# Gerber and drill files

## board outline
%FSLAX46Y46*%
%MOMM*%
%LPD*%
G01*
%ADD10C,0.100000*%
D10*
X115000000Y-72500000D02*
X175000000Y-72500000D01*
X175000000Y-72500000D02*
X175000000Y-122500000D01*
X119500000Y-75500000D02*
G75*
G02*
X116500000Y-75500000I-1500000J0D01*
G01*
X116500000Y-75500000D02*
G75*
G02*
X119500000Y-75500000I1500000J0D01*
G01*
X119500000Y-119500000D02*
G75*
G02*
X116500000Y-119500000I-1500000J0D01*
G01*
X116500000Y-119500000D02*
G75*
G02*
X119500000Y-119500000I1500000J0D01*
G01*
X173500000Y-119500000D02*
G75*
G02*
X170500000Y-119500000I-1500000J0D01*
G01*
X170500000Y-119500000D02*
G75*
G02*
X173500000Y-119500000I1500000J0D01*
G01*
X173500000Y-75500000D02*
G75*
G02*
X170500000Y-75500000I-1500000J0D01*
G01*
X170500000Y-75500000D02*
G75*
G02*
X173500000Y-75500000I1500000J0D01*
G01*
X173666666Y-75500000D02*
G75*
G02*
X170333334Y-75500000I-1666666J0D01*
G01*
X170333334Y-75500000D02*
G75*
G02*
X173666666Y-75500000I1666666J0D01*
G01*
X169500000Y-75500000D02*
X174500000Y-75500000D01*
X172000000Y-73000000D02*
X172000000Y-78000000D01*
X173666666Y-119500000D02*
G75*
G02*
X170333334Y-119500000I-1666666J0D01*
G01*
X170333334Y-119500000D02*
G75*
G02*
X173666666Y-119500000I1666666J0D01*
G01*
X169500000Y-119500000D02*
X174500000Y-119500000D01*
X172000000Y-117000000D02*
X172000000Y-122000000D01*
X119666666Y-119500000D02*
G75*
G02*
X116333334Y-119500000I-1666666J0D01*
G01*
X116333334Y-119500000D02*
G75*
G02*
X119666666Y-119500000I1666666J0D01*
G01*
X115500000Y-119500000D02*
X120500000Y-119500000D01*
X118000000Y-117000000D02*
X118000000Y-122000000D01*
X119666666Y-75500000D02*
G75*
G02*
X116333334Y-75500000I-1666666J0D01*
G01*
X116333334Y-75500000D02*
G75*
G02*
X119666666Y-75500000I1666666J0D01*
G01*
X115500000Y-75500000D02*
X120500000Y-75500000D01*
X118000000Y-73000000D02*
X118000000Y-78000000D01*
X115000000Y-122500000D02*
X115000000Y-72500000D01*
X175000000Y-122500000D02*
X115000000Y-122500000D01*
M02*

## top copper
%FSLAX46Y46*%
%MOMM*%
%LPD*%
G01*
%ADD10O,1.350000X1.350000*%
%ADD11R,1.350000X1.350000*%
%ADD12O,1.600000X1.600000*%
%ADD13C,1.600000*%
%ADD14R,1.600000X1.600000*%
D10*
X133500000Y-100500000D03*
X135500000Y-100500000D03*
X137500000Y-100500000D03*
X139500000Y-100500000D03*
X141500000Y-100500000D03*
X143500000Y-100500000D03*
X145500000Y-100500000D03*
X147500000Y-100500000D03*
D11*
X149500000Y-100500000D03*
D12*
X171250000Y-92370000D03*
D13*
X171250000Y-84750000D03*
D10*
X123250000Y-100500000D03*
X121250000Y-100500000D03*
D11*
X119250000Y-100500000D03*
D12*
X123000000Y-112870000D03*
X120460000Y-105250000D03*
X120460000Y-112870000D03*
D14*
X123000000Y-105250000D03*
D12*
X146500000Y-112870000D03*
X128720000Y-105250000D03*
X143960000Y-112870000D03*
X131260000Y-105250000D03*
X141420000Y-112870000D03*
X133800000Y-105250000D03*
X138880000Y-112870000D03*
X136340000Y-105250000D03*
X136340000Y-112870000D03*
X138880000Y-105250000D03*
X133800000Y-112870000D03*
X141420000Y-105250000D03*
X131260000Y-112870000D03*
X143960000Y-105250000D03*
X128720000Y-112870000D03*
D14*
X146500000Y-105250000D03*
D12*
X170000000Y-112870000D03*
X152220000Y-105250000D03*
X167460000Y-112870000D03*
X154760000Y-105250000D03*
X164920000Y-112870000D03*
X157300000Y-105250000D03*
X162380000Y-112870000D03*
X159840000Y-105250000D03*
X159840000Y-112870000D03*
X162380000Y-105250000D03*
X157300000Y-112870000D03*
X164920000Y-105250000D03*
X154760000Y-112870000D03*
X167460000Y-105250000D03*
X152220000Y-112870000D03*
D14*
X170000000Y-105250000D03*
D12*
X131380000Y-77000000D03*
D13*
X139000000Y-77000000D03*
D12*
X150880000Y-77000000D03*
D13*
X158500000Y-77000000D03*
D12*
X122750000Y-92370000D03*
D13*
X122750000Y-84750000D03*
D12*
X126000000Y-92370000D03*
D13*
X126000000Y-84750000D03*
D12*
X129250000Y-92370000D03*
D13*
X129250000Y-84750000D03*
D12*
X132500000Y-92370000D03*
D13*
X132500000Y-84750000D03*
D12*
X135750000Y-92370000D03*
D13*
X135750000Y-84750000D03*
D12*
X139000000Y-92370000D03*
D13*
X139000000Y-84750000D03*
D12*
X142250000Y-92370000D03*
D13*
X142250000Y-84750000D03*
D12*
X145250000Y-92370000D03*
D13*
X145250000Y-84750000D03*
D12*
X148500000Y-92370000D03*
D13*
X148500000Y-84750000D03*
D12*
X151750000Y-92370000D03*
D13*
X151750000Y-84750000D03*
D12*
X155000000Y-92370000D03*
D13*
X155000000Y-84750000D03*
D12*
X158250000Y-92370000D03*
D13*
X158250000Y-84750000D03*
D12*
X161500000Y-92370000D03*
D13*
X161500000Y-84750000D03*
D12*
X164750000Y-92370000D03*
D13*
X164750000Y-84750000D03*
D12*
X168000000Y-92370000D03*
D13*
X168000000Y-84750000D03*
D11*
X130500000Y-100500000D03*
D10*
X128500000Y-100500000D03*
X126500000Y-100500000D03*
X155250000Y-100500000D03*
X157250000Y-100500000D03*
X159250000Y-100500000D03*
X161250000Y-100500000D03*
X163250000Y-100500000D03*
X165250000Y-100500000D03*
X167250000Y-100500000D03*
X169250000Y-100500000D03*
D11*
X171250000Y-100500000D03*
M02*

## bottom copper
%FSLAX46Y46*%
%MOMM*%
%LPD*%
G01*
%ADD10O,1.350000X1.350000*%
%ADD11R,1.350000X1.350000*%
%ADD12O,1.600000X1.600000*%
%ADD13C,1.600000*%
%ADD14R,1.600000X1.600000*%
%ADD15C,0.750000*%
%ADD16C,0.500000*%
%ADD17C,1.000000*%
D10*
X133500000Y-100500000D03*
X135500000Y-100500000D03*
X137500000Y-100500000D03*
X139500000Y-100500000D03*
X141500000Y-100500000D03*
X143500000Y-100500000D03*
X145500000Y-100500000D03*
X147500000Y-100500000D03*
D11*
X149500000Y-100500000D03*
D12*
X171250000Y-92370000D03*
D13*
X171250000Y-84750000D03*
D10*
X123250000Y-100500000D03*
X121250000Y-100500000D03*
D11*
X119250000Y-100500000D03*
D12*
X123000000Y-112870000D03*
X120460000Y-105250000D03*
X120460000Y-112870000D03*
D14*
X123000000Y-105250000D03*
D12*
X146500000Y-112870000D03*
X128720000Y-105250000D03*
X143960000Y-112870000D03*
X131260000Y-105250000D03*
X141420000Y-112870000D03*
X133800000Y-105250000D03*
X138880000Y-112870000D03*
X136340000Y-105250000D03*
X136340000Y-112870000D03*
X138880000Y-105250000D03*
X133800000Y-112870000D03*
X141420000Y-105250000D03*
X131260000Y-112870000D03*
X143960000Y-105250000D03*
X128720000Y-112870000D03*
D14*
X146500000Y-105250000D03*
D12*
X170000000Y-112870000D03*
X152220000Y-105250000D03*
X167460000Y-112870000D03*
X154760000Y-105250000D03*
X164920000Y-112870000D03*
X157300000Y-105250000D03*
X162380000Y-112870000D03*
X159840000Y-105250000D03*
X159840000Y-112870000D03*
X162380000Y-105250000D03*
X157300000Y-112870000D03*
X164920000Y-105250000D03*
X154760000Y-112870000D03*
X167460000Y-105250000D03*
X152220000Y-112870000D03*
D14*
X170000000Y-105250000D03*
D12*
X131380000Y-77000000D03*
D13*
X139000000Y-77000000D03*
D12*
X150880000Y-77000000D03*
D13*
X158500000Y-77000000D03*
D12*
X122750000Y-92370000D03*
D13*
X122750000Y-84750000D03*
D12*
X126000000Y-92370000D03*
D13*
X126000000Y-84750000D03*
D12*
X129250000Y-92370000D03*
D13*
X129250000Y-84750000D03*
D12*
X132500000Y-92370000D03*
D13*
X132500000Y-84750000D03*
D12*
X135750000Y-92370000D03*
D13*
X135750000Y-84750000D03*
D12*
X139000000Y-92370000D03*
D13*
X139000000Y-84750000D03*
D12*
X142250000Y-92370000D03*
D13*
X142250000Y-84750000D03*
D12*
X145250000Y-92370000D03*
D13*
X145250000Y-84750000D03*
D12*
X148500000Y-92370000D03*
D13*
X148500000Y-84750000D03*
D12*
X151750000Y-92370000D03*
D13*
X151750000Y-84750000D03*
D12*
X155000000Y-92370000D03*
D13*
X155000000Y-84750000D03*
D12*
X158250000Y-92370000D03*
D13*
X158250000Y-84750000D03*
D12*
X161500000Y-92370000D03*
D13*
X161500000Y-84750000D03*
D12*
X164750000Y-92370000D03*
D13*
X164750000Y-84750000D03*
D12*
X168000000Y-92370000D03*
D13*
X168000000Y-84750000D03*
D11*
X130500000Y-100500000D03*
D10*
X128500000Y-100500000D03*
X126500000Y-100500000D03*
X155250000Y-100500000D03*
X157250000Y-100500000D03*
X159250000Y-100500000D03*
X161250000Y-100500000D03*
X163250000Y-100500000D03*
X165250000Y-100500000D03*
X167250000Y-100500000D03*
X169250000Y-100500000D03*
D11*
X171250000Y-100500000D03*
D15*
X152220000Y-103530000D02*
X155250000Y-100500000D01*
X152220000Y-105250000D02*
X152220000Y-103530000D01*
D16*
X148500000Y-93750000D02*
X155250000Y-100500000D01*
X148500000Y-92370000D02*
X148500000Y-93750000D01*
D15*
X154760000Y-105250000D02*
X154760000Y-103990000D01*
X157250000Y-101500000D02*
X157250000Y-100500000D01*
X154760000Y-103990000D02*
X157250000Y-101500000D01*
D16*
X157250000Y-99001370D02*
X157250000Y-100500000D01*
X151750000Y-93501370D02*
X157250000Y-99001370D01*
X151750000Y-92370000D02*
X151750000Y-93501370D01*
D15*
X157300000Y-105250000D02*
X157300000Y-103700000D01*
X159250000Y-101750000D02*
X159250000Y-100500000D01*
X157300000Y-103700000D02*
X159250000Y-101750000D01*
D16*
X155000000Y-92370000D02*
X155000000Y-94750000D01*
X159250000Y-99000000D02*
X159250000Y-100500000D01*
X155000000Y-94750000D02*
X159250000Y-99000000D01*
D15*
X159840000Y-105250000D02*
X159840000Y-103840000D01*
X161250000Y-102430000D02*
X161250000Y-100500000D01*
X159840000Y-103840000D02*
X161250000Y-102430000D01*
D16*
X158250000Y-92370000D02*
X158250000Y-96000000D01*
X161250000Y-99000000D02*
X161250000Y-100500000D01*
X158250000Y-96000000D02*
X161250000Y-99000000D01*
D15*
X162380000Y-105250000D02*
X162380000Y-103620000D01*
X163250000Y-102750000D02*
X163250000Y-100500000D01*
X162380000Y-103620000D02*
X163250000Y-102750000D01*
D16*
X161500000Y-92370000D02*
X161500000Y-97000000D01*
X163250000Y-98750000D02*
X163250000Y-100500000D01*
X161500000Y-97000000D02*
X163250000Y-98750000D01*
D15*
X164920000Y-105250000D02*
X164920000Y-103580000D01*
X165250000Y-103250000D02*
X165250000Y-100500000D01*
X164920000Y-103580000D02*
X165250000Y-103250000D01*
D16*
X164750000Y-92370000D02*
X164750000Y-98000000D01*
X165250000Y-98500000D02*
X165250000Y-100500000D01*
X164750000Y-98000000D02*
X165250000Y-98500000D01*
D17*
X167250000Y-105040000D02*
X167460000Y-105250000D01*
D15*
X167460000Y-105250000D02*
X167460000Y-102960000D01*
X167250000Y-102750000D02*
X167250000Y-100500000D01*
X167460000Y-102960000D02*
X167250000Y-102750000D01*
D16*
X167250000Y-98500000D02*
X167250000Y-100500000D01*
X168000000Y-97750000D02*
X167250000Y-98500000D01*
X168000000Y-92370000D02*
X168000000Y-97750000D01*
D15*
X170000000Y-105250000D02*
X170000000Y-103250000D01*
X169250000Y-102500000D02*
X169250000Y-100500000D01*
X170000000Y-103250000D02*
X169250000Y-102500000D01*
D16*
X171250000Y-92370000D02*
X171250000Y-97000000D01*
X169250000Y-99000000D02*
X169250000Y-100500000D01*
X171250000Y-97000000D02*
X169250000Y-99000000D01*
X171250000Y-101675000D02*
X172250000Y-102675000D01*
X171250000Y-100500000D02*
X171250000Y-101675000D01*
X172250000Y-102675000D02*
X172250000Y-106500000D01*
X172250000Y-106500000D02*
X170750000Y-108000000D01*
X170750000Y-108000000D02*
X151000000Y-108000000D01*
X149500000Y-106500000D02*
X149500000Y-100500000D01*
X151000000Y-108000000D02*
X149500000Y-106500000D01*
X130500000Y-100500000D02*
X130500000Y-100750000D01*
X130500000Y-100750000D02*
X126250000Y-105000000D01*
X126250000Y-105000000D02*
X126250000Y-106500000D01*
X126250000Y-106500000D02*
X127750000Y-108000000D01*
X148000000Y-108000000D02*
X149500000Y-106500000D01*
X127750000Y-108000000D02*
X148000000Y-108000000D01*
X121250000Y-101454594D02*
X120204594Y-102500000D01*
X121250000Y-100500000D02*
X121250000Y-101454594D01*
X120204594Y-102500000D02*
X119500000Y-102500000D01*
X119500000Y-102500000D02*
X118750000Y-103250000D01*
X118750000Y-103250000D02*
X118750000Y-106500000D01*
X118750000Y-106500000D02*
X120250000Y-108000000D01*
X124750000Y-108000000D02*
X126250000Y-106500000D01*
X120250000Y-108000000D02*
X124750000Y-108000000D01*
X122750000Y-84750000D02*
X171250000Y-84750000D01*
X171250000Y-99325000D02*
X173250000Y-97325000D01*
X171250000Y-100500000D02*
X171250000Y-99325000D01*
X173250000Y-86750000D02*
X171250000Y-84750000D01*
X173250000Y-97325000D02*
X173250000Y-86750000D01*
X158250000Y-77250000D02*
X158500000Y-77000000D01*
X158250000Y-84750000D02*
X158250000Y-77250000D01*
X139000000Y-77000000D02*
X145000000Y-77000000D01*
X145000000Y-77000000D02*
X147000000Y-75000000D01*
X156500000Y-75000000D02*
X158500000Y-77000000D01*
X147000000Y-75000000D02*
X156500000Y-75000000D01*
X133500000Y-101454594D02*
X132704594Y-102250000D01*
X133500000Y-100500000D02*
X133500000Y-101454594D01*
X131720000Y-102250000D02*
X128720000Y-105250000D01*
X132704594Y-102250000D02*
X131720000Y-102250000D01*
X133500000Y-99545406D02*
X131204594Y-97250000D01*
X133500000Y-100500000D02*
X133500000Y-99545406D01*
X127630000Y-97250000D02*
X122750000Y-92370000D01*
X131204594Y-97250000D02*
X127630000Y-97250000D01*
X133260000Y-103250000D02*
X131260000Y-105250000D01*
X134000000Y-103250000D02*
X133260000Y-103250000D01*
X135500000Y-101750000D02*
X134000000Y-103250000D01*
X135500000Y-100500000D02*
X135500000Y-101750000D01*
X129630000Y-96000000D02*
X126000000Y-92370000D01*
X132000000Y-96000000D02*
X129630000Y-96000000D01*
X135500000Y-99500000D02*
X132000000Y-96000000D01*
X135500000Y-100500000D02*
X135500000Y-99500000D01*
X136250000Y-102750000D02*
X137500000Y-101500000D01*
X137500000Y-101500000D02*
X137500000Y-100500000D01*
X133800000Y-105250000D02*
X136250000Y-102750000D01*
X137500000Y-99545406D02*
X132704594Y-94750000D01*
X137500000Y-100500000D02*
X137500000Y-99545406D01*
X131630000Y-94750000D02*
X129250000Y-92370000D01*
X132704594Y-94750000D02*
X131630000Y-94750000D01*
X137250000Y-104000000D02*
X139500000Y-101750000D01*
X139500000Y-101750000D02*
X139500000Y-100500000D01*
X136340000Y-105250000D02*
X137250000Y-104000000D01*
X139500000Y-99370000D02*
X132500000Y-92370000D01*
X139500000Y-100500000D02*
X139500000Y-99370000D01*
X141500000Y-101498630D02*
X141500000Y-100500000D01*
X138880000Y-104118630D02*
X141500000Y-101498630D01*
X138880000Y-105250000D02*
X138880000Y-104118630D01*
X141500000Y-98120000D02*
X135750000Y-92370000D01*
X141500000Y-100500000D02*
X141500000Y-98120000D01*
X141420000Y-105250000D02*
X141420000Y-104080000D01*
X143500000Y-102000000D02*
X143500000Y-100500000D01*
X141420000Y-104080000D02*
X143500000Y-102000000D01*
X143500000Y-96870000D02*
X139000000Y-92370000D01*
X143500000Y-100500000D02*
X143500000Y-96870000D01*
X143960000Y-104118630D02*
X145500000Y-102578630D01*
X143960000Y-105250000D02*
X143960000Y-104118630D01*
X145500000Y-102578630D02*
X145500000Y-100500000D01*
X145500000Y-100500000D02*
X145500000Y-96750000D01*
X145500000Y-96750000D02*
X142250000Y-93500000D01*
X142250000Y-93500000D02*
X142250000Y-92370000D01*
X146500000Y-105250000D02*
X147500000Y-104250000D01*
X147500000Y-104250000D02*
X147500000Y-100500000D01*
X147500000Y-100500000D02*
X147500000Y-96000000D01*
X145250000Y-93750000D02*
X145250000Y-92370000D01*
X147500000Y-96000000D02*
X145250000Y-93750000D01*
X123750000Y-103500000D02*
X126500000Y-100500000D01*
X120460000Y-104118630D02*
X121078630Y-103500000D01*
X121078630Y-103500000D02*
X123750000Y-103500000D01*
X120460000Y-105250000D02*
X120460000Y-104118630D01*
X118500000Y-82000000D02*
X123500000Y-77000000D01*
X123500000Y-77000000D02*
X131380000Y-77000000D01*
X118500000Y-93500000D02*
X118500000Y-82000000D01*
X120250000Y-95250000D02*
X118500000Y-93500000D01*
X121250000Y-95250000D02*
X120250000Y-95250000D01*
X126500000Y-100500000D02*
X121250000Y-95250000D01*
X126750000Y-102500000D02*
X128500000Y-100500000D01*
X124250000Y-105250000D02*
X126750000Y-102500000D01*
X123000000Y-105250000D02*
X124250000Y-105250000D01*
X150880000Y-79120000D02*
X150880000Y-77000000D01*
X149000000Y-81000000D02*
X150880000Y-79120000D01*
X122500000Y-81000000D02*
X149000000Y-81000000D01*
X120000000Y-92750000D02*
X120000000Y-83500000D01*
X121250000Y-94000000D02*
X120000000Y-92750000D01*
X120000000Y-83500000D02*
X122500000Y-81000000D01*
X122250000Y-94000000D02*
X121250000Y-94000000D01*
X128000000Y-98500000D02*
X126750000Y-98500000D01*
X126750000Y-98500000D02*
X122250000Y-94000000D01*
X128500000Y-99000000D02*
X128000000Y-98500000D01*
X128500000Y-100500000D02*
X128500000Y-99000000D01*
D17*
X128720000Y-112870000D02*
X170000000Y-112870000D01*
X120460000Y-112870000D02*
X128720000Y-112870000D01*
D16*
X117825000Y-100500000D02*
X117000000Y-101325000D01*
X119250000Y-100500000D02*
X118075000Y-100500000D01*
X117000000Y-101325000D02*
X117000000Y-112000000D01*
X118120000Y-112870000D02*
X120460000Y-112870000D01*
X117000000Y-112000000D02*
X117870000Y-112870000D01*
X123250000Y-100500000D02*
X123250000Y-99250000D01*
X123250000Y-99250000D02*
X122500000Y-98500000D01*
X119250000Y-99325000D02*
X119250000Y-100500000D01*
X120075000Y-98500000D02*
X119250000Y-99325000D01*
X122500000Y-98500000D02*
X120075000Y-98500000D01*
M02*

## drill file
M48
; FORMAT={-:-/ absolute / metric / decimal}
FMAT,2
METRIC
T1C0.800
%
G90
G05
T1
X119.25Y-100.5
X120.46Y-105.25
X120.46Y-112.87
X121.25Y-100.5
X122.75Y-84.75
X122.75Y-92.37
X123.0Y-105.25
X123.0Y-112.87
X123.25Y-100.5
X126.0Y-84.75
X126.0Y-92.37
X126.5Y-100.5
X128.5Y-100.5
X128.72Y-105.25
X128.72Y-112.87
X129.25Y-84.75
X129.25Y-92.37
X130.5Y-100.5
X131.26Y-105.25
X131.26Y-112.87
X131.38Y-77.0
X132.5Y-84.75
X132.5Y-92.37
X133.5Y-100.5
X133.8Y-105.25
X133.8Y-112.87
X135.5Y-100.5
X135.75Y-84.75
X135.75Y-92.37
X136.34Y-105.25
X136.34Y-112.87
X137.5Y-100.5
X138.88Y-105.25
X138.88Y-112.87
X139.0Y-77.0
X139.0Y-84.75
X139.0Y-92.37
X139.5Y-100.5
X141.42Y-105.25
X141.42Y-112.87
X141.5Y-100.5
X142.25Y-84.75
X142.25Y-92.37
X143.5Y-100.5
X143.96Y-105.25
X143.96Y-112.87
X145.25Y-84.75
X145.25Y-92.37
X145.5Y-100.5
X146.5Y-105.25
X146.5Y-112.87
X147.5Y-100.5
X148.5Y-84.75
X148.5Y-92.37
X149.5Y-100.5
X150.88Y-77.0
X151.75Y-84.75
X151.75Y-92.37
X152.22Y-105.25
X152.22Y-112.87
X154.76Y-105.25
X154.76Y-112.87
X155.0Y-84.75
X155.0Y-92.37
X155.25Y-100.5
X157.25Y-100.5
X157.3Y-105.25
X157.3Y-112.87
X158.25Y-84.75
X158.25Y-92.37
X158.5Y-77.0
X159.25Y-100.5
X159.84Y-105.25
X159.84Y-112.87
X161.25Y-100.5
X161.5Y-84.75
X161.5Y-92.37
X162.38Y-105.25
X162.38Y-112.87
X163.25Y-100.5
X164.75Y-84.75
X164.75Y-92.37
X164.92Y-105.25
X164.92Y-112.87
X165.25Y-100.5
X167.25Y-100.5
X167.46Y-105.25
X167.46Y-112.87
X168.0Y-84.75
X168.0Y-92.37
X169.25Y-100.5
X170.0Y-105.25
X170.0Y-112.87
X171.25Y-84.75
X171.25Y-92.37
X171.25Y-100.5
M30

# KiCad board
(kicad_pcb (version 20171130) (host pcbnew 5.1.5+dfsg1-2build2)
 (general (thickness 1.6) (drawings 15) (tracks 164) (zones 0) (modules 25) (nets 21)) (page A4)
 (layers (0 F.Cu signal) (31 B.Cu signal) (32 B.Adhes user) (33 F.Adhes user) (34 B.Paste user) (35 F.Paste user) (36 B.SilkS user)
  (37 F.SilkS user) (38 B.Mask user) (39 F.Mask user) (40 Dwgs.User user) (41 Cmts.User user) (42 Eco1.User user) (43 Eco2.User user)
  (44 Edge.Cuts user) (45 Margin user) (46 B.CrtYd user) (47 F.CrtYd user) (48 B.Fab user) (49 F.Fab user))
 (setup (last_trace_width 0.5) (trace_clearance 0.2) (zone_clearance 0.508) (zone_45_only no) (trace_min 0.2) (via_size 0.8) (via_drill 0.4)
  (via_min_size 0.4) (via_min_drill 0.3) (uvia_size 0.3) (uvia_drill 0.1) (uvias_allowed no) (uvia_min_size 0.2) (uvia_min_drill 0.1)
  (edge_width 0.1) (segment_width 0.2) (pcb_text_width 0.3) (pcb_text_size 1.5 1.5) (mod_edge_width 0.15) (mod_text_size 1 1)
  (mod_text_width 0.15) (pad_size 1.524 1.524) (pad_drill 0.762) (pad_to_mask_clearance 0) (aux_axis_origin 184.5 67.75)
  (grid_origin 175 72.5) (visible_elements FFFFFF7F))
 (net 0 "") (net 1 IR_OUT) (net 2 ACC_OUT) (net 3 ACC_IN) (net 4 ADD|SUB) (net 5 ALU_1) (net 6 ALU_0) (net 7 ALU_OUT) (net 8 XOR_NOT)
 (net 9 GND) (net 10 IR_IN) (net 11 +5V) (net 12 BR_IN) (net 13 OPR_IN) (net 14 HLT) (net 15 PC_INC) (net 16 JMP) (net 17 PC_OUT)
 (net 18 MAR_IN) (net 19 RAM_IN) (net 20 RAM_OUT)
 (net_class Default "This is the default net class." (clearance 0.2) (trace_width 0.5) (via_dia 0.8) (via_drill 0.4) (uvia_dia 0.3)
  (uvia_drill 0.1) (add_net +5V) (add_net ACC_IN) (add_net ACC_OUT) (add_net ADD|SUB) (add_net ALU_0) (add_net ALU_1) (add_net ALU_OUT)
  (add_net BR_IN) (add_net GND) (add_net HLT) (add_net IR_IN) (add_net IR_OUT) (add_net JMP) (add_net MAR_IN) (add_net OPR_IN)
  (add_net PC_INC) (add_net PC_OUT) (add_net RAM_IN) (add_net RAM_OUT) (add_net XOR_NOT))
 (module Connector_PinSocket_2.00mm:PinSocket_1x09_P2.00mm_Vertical (layer F.Cu) (at 149.5 100.5 270)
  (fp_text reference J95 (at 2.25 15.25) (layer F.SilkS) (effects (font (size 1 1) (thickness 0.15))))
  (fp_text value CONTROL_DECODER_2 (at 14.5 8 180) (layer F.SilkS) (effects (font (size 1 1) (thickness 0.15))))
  (pad 9 thru_hole oval (at 0 16 270) (size 1.35 1.35) (drill 0.8) (layers *.Cu *.Mask) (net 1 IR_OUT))
  (pad 8 thru_hole oval (at 0 14 270) (size 1.35 1.35) (drill 0.8) (layers *.Cu *.Mask) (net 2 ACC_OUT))
  (pad 7 thru_hole oval (at 0 12 270) (size 1.35 1.35) (drill 0.8) (layers *.Cu *.Mask) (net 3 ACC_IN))
  (pad 6 thru_hole oval (at 0 10 270) (size 1.35 1.35) (drill 0.8) (layers *.Cu *.Mask) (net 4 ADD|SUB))
  (pad 5 thru_hole oval (at 0 8 270) (size 1.35 1.35) (drill 0.8) (layers *.Cu *.Mask) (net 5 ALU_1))
  (pad 4 thru_hole oval (at 0 6 270) (size 1.35 1.35) (drill 0.8) (layers *.Cu *.Mask) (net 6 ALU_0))
  (pad 3 thru_hole oval (at 0 4 270) (size 1.35 1.35) (drill 0.8) (layers *.Cu *.Mask) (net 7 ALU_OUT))
  (pad 2 thru_hole oval (at 0 2 270) (size 1.35 1.35) (drill 0.8) (layers *.Cu *.Mask) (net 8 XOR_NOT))
  (pad 1 thru_hole rect (at 0 0 270) (size 1.35 1.35) (drill 0.8) (layers *.Cu *.Mask) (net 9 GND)))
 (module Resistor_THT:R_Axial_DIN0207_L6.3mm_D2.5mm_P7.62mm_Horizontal (layer F.Cu) (at 171.25 84.75 270)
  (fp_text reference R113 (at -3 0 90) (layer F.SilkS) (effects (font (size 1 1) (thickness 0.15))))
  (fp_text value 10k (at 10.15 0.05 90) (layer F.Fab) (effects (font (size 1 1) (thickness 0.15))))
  (pad 2 thru_hole oval (at 7.62 0 270) (size 1.6 1.6) (drill 0.8) (layers *.Cu *.Mask) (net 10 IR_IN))
  (pad 1 thru_hole circle (at 0 0 270) (size 1.6 1.6) (drill 0.8) (layers *.Cu *.Mask) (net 9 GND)))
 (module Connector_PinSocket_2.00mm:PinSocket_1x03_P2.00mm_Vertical (layer F.Cu) (at 119.25 100.5 90)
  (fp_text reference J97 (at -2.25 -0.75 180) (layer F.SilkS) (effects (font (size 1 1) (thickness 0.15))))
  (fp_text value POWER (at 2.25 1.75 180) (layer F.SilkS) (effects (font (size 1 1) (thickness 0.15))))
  (pad 3 thru_hole oval (at 0 4 90) (size 1.35 1.35) (drill 0.8) (layers *.Cu *.Mask) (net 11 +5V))
  (pad 2 thru_hole oval (at 0 2 90) (size 1.35 1.35) (drill 0.8) (layers *.Cu *.Mask) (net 9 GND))
  (pad 1 thru_hole rect (at 0 0 90) (size 1.35 1.35) (drill 0.8) (layers *.Cu *.Mask) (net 11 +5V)))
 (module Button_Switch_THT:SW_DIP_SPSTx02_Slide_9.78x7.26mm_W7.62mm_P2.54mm (layer F.Cu) (at 123 105.25 270)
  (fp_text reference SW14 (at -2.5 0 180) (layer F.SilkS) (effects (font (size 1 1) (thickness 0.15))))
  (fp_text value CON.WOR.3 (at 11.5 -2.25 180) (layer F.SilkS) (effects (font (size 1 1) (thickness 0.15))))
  (pad 4 thru_hole oval (at 7.62 0 270) (size 1.6 1.6) (drill 0.8) (layers *.Cu *.Mask) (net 11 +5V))
  (pad 2 thru_hole oval (at 0 2.54 270) (size 1.6 1.6) (drill 0.8) (layers *.Cu *.Mask) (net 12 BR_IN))
  (pad 3 thru_hole oval (at 7.62 2.54 270) (size 1.6 1.6) (drill 0.8) (layers *.Cu *.Mask) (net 11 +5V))
  (pad 1 thru_hole rect (at 0 0 270) (size 1.6 1.6) (drill 0.8) (layers *.Cu *.Mask) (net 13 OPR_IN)))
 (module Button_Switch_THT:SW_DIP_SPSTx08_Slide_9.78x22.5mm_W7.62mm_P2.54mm (layer F.Cu) (at 146.5 105.25 270)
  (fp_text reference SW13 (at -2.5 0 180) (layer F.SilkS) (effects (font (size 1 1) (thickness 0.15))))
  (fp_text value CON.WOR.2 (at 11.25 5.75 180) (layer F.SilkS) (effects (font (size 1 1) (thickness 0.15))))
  (pad 16 thru_hole oval (at 7.62 0 270) (size 1.6 1.6) (drill 0.8) (layers *.Cu *.Mask) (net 11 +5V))
  (pad 8 thru_hole oval (at 0 17.78 270) (size 1.6 1.6) (drill 0.8) (layers *.Cu *.Mask) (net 1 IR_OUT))
  (pad 15 thru_hole oval (at 7.62 2.54 270) (size 1.6 1.6) (drill 0.8) (layers *.Cu *.Mask) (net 11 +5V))
  (pad 7 thru_hole oval (at 0 15.24 270) (size 1.6 1.6) (drill 0.8) (layers *.Cu *.Mask) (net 2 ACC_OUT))
  (pad 14 thru_hole oval (at 7.62 5.08 270) (size 1.6 1.6) (drill 0.8) (layers *.Cu *.Mask) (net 11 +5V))
  (pad 6 thru_hole oval (at 0 12.7 270) (size 1.6 1.6) (drill 0.8) (layers *.Cu *.Mask) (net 3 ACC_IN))
  (pad 13 thru_hole oval (at 7.62 7.62 270) (size 1.6 1.6) (drill 0.8) (layers *.Cu *.Mask) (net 11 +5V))
  (pad 5 thru_hole oval (at 0 10.16 270) (size 1.6 1.6) (drill 0.8) (layers *.Cu *.Mask) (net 4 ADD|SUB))
  (pad 12 thru_hole oval (at 7.62 10.16 270) (size 1.6 1.6) (drill 0.8) (layers *.Cu *.Mask) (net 11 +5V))
  (pad 4 thru_hole oval (at 0 7.62 270) (size 1.6 1.6) (drill 0.8) (layers *.Cu *.Mask) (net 5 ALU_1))
  (pad 11 thru_hole oval (at 7.62 12.7 270) (size 1.6 1.6) (drill 0.8) (layers *.Cu *.Mask) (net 11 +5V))
  (pad 3 thru_hole oval (at 0 5.08 270) (size 1.6 1.6) (drill 0.8) (layers *.Cu *.Mask) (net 6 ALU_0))
  (pad 10 thru_hole oval (at 7.62 15.24 270) (size 1.6 1.6) (drill 0.8) (layers *.Cu *.Mask) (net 11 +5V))
  (pad 2 thru_hole oval (at 0 2.54 270) (size 1.6 1.6) (drill 0.8) (layers *.Cu *.Mask) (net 7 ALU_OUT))
  (pad 9 thru_hole oval (at 7.62 17.78 270) (size 1.6 1.6) (drill 0.8) (layers *.Cu *.Mask) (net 11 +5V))
  (pad 1 thru_hole rect (at 0 0 270) (size 1.6 1.6) (drill 0.8) (layers *.Cu *.Mask) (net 8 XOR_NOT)))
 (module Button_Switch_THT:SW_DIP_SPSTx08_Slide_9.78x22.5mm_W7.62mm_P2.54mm (layer F.Cu) (at 170 105.25 270)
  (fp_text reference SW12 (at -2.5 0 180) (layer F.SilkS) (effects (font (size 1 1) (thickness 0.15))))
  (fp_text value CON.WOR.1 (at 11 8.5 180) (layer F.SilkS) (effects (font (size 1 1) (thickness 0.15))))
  (pad 16 thru_hole oval (at 7.62 0 270) (size 1.6 1.6) (drill 0.8) (layers *.Cu *.Mask) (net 11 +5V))
  (pad 8 thru_hole oval (at 0 17.78 270) (size 1.6 1.6) (drill 0.8) (layers *.Cu *.Mask) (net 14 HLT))
  (pad 15 thru_hole oval (at 7.62 2.54 270) (size 1.6 1.6) (drill 0.8) (layers *.Cu *.Mask) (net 11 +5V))
  (pad 7 thru_hole oval (at 0 15.24 270) (size 1.6 1.6) (drill 0.8) (layers *.Cu *.Mask) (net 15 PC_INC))
  (pad 14 thru_hole oval (at 7.62 5.08 270) (size 1.6 1.6) (drill 0.8) (layers *.Cu *.Mask) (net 11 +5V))
  (pad 6 thru_hole oval (at 0 12.7 270) (size 1.6 1.6) (drill 0.8) (layers *.Cu *.Mask) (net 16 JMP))
  (pad 13 thru_hole oval (at 7.62 7.62 270) (size 1.6 1.6) (drill 0.8) (layers *.Cu *.Mask) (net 11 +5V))
  (pad 5 thru_hole oval (at 0 10.16 270) (size 1.6 1.6) (drill 0.8) (layers *.Cu *.Mask) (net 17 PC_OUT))
  (pad 12 thru_hole oval (at 7.62 10.16 270) (size 1.6 1.6) (drill 0.8) (layers *.Cu *.Mask) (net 11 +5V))
  (pad 4 thru_hole oval (at 0 7.62 270) (size 1.6 1.6) (drill 0.8) (layers *.Cu *.Mask) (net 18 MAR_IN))
  (pad 11 thru_hole oval (at 7.62 12.7 270) (size 1.6 1.6) (drill 0.8) (layers *.Cu *.Mask) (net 11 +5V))
  (pad 3 thru_hole oval (at 0 5.08 270) (size 1.6 1.6) (drill 0.8) (layers *.Cu *.Mask) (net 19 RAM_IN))
  (pad 10 thru_hole oval (at 7.62 15.24 270) (size 1.6 1.6) (drill 0.8) (layers *.Cu *.Mask) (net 11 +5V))
  (pad 2 thru_hole oval (at 0 2.54 270) (size 1.6 1.6) (drill 0.8) (layers *.Cu *.Mask) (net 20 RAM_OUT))
  (pad 9 thru_hole oval (at 7.62 17.78 270) (size 1.6 1.6) (drill 0.8) (layers *.Cu *.Mask) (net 11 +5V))
  (pad 1 thru_hole rect (at 0 0 270) (size 1.6 1.6) (drill 0.8) (layers *.Cu *.Mask) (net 10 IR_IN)))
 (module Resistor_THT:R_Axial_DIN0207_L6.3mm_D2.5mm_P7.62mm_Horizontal (layer F.Cu) (at 139 77 180)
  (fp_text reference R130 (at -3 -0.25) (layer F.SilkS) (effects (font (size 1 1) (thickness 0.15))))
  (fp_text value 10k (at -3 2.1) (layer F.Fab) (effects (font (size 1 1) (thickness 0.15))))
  (pad 2 thru_hole oval (at 7.62 0 180) (size 1.6 1.6) (drill 0.8) (layers *.Cu *.Mask) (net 12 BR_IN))
  (pad 1 thru_hole circle (at 0 0 180) (size 1.6 1.6) (drill 0.8) (layers *.Cu *.Mask) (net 9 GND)))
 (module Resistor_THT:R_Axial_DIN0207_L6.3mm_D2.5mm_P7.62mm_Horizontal (layer F.Cu) (at 158.5 77 180)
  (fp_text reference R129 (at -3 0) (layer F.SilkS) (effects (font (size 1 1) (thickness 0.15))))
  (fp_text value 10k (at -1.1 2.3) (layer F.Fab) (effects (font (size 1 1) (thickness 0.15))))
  (pad 2 thru_hole oval (at 7.62 0 180) (size 1.6 1.6) (drill 0.8) (layers *.Cu *.Mask) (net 13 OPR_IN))
  (pad 1 thru_hole circle (at 0 0 180) (size 1.6 1.6) (drill 0.8) (layers *.Cu *.Mask) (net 9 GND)))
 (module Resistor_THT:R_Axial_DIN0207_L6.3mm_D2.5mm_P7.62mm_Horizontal (layer F.Cu) (at 122.75 84.75 270)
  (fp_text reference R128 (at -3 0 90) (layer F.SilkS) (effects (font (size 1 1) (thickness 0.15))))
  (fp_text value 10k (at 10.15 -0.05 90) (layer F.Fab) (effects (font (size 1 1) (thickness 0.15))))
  (pad 2 thru_hole oval (at 7.62 0 270) (size 1.6 1.6) (drill 0.8) (layers *.Cu *.Mask) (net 1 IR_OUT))
  (pad 1 thru_hole circle (at 0 0 270) (size 1.6 1.6) (drill 0.8) (layers *.Cu *.Mask) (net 9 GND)))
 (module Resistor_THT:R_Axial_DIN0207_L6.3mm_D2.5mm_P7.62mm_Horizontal (layer F.Cu) (at 126 84.75 270)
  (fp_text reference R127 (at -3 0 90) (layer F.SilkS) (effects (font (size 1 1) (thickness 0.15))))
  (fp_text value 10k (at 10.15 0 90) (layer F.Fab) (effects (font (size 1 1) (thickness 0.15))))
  (pad 2 thru_hole oval (at 7.62 0 270) (size 1.6 1.6) (drill 0.8) (layers *.Cu *.Mask) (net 2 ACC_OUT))
  (pad 1 thru_hole circle (at 0 0 270) (size 1.6 1.6) (drill 0.8) (layers *.Cu *.Mask) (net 9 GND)))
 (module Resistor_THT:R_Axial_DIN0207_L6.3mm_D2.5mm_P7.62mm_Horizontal (layer F.Cu) (at 129.25 84.75 270)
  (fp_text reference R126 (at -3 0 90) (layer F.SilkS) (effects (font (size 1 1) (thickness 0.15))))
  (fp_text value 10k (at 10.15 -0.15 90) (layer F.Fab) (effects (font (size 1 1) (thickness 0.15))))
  (pad 2 thru_hole oval (at 7.62 0 270) (size 1.6 1.6) (drill 0.8) (layers *.Cu *.Mask) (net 3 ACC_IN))
  (pad 1 thru_hole circle (at 0 0 270) (size 1.6 1.6) (drill 0.8) (layers *.Cu *.Mask) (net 9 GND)))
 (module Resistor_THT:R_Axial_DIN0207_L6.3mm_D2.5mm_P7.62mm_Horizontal (layer F.Cu) (at 132.5 84.75 270)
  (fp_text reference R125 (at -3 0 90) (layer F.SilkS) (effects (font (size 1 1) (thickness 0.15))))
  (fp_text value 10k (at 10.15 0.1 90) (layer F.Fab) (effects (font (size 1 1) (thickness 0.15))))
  (pad 2 thru_hole oval (at 7.62 0 270) (size 1.6 1.6) (drill 0.8) (layers *.Cu *.Mask) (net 4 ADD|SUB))
  (pad 1 thru_hole circle (at 0 0 270) (size 1.6 1.6) (drill 0.8) (layers *.Cu *.Mask) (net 9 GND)))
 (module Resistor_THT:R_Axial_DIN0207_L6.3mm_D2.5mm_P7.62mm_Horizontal (layer F.Cu) (at 135.75 84.75 270)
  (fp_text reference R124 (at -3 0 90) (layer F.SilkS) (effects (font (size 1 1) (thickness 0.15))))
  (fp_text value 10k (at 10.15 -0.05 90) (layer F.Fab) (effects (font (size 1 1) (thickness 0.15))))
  (pad 2 thru_hole oval (at 7.62 0 270) (size 1.6 1.6) (drill 0.8) (layers *.Cu *.Mask) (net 5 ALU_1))
  (pad 1 thru_hole circle (at 0 0 270) (size 1.6 1.6) (drill 0.8) (layers *.Cu *.Mask) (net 9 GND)))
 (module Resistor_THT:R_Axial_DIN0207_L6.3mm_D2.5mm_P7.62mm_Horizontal (layer F.Cu) (at 139 84.75 270)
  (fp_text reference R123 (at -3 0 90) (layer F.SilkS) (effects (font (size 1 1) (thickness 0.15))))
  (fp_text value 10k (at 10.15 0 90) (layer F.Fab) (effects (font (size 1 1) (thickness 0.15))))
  (pad 2 thru_hole oval (at 7.62 0 270) (size 1.6 1.6) (drill 0.8) (layers *.Cu *.Mask) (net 6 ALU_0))
  (pad 1 thru_hole circle (at 0 0 270) (size 1.6 1.6) (drill 0.8) (layers *.Cu *.Mask) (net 9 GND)))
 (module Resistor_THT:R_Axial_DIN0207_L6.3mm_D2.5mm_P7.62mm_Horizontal (layer F.Cu) (at 142.25 84.75 270)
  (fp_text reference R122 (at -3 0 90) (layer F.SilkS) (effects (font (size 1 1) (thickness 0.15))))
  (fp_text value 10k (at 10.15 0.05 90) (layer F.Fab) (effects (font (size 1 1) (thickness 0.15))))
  (pad 2 thru_hole oval (at 7.62 0 270) (size 1.6 1.6) (drill 0.8) (layers *.Cu *.Mask) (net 7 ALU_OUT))
  (pad 1 thru_hole circle (at 0 0 270) (size 1.6 1.6) (drill 0.8) (layers *.Cu *.Mask) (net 9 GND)))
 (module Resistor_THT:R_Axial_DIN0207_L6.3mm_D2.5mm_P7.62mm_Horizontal (layer F.Cu) (at 145.25 84.75 270)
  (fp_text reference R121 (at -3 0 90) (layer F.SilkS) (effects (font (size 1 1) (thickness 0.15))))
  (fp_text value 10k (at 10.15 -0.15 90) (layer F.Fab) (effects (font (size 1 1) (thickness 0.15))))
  (pad 2 thru_hole oval (at 7.62 0 270) (size 1.6 1.6) (drill 0.8) (layers *.Cu *.Mask) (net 8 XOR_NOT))
  (pad 1 thru_hole circle (at 0 0 270) (size 1.6 1.6) (drill 0.8) (layers *.Cu *.Mask) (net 9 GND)))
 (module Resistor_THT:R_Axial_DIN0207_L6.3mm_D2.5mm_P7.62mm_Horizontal (layer F.Cu) (at 148.5 84.75 270)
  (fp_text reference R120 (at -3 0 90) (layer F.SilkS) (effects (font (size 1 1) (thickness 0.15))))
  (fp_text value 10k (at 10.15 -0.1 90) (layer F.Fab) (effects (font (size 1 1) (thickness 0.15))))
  (pad 2 thru_hole oval (at 7.62 0 270) (size 1.6 1.6) (drill 0.8) (layers *.Cu *.Mask) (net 14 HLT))
  (pad 1 thru_hole circle (at 0 0 270) (size 1.6 1.6) (drill 0.8) (layers *.Cu *.Mask) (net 9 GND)))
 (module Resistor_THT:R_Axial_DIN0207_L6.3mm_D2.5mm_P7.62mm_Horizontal (layer F.Cu) (at 151.75 84.75 270)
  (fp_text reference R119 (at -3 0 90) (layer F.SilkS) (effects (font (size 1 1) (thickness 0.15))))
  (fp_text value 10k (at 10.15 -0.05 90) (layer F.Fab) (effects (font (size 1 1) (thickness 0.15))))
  (pad 2 thru_hole oval (at 7.62 0 270) (size 1.6 1.6) (drill 0.8) (layers *.Cu *.Mask) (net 15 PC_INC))
  (pad 1 thru_hole circle (at 0 0 270) (size 1.6 1.6) (drill 0.8) (layers *.Cu *.Mask) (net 9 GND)))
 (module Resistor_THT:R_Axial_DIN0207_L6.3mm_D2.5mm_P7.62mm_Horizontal (layer F.Cu) (at 155 84.75 270)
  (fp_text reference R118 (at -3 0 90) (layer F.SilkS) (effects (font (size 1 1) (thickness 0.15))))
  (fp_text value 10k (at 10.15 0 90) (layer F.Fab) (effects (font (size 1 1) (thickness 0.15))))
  (pad 2 thru_hole oval (at 7.62 0 270) (size 1.6 1.6) (drill 0.8) (layers *.Cu *.Mask) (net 16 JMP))
  (pad 1 thru_hole circle (at 0 0 270) (size 1.6 1.6) (drill 0.8) (layers *.Cu *.Mask) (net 9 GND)))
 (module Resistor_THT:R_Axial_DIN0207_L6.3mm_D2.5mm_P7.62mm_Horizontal (layer F.Cu) (at 158.25 84.75 270)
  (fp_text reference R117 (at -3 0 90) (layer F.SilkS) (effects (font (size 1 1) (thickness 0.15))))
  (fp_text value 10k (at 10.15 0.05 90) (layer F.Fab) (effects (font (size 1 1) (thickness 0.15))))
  (pad 2 thru_hole oval (at 7.62 0 270) (size 1.6 1.6) (drill 0.8) (layers *.Cu *.Mask) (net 17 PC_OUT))
  (pad 1 thru_hole circle (at 0 0 270) (size 1.6 1.6) (drill 0.8) (layers *.Cu *.Mask) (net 9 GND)))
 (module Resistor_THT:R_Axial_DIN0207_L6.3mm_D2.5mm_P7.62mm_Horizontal (layer F.Cu) (at 161.5 84.75 270)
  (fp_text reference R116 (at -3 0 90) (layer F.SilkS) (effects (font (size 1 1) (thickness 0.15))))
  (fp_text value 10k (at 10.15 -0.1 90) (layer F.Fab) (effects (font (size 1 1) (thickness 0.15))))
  (pad 2 thru_hole oval (at 7.62 0 270) (size 1.6 1.6) (drill 0.8) (layers *.Cu *.Mask) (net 18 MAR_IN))
  (pad 1 thru_hole circle (at 0 0 270) (size 1.6 1.6) (drill 0.8) (layers *.Cu *.Mask) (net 9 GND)))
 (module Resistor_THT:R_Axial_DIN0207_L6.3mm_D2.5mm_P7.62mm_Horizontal (layer F.Cu) (at 164.75 84.75 270)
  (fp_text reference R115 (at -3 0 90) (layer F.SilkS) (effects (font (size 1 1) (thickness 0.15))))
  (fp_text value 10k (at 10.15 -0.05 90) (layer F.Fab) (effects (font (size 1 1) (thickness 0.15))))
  (pad 2 thru_hole oval (at 7.62 0 270) (size 1.6 1.6) (drill 0.8) (layers *.Cu *.Mask) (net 19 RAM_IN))
  (pad 1 thru_hole circle (at 0 0 270) (size 1.6 1.6) (drill 0.8) (layers *.Cu *.Mask) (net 9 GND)))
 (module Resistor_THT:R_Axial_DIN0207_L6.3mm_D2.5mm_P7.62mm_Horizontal (layer F.Cu) (at 168 84.75 270)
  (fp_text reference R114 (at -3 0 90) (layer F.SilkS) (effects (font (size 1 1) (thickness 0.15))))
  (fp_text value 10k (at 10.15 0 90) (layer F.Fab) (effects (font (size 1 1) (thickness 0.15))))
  (pad 2 thru_hole oval (at 7.62 0 270) (size 1.6 1.6) (drill 0.8) (layers *.Cu *.Mask) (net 20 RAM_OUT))
  (pad 1 thru_hole circle (at 0 0 270) (size 1.6 1.6) (drill 0.8) (layers *.Cu *.Mask) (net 9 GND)))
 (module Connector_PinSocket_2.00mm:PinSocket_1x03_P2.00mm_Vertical (layer F.Cu) (at 130.5 100.5 270)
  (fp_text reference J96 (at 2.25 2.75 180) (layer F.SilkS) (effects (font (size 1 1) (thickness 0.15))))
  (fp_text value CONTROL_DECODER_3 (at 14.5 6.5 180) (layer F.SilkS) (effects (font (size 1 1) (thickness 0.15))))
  (pad 1 thru_hole rect (at 0 0 270) (size 1.35 1.35) (drill 0.8) (layers *.Cu *.Mask) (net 9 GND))
  (pad 2 thru_hole oval (at 0 2 270) (size 1.35 1.35) (drill 0.8) (layers *.Cu *.Mask) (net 13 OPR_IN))
  (pad 3 thru_hole oval (at 0 4 270) (size 1.35 1.35) (drill 0.8) (layers *.Cu *.Mask) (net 12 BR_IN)))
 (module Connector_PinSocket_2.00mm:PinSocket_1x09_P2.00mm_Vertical (layer F.Cu) (at 171.25 100.5 270)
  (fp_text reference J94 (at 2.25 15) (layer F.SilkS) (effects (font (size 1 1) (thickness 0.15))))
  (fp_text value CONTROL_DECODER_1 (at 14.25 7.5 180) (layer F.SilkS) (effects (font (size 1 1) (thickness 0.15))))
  (pad 9 thru_hole oval (at 0 16 270) (size 1.35 1.35) (drill 0.8) (layers *.Cu *.Mask) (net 14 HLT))
  (pad 8 thru_hole oval (at 0 14 270) (size 1.35 1.35) (drill 0.8) (layers *.Cu *.Mask) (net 15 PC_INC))
  (pad 7 thru_hole oval (at 0 12 270) (size 1.35 1.35) (drill 0.8) (layers *.Cu *.Mask) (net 16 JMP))
  (pad 6 thru_hole oval (at 0 10 270) (size 1.35 1.35) (drill 0.8) (layers *.Cu *.Mask) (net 17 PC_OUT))
  (pad 5 thru_hole oval (at 0 8 270) (size 1.35 1.35) (drill 0.8) (layers *.Cu *.Mask) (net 18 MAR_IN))
  (pad 4 thru_hole oval (at 0 6 270) (size 1.35 1.35) (drill 0.8) (layers *.Cu *.Mask) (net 19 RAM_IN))
  (pad 3 thru_hole oval (at 0 4 270) (size 1.35 1.35) (drill 0.8) (layers *.Cu *.Mask) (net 20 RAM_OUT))
  (pad 2 thru_hole oval (at 0 2 270) (size 1.35 1.35) (drill 0.8) (layers *.Cu *.Mask) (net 10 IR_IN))
  (pad 1 thru_hole rect (at 0 0 270) (size 1.35 1.35) (drill 0.8) (layers *.Cu *.Mask) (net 9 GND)))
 (gr_line (start 115 72.5) (end 175 72.5) (layer Edge.Cuts) (width 0.1))
 (gr_line (start 175 72.5) (end 175 122.5) (layer Edge.Cuts) (width 0.1))
 (gr_circle (center 118 75.5) (end 119.5 75.5) (layer Edge.Cuts) (width 0.1))
 (gr_circle (center 118 119.5) (end 119.5 119.5) (layer Edge.Cuts) (width 0.1))
 (gr_circle (center 172 119.5) (end 173.5 119.5) (layer Edge.Cuts) (width 0.1))
 (gr_circle (center 172 75.5) (end 173.5 75.5) (layer Edge.Cuts) (width 0.1))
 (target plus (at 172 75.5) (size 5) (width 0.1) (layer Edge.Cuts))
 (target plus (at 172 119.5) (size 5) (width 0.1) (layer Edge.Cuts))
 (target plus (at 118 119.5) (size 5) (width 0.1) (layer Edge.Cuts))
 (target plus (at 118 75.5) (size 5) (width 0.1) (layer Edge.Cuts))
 (gr_line (start 115 122.5) (end 115 72.5) (layer Edge.Cuts) (width 0.1))
 (gr_line (start 175 122.5) (end 115 122.5) (layer Edge.Cuts) (width 0.1))
 (segment (start 152.22 103.53) (end 155.25 100.5) (width 0.75) (layer B.Cu) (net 14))
 (segment (start 152.22 105.25) (end 152.22 103.53) (width 0.75) (layer B.Cu) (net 14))
 (segment (start 148.5 93.75) (end 155.25 100.5) (width 0.5) (layer B.Cu) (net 14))
 (segment (start 148.5 92.37) (end 148.5 93.75) (width 0.5) (layer B.Cu) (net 14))
 (segment (start 154.76 105.25) (end 154.76 103.99) (width 0.75) (layer B.Cu) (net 15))
 (segment (start 157.25 101.5) (end 157.25 100.5) (width 0.75) (layer B.Cu) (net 15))
 (segment (start 154.76 103.99) (end 157.25 101.5) (width 0.75) (layer B.Cu) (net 15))
 (segment (start 157.25 99.00137) (end 157.25 100.5) (width 0.5) (layer B.Cu) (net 15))
 (segment (start 151.75 93.50137) (end 157.25 99.00137) (width 0.5) (layer B.Cu) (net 15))
 (segment (start 151.75 92.37) (end 151.75 93.50137) (width 0.5) (layer B.Cu) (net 15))
 (segment (start 157.3 105.25) (end 157.3 103.7) (width 0.75) (layer B.Cu) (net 16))
 (segment (start 159.25 101.75) (end 159.25 100.5) (width 0.75) (layer B.Cu) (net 16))
 (segment (start 157.3 103.7) (end 159.25 101.75) (width 0.75) (layer B.Cu) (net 16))
 (segment (start 155 92.37) (end 155 94.75) (width 0.5) (layer B.Cu) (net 16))
 (segment (start 159.25 99) (end 159.25 100.5) (width 0.5) (layer B.Cu) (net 16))
 (segment (start 155 94.75) (end 159.25 99) (width 0.5) (layer B.Cu) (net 16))
 (segment (start 159.84 105.25) (end 159.84 103.84) (width 0.75) (layer B.Cu) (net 17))
 (segment (start 161.25 102.43) (end 161.25 100.5) (width 0.75) (layer B.Cu) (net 17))
 (segment (start 159.84 103.84) (end 161.25 102.43) (width 0.75) (layer B.Cu) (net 17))
 (segment (start 158.25 92.37) (end 158.25 96) (width 0.5) (layer B.Cu) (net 17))
 (segment (start 161.25 99) (end 161.25 100.5) (width 0.5) (layer B.Cu) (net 17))
 (segment (start 158.25 96) (end 161.25 99) (width 0.5) (layer B.Cu) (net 17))
 (segment (start 162.38 105.25) (end 162.38 103.62) (width 0.75) (layer B.Cu) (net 18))
 (segment (start 163.25 102.75) (end 163.25 100.5) (width 0.75) (layer B.Cu) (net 18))
 (segment (start 162.38 103.62) (end 163.25 102.75) (width 0.75) (layer B.Cu) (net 18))
 (segment (start 161.5 92.37) (end 161.5 97) (width 0.5) (layer B.Cu) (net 18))
 (segment (start 163.25 98.75) (end 163.25 100.5) (width 0.5) (layer B.Cu) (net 18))
 (segment (start 161.5 97) (end 163.25 98.75) (width 0.5) (layer B.Cu) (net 18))
 (segment (start 164.92 105.25) (end 164.92 103.58) (width 0.75) (layer B.Cu) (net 19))
 (segment (start 165.25 103.25) (end 165.25 100.5) (width 0.75) (layer B.Cu) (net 19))
 (segment (start 164.92 103.58) (end 165.25 103.25) (width 0.75) (layer B.Cu) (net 19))
 (segment (start 164.75 92.37) (end 164.75 98) (width 0.5) (layer B.Cu) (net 19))
 (segment (start 165.25 98.5) (end 165.25 100.5) (width 0.5) (layer B.Cu) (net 19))
 (segment (start 164.75 98) (end 165.25 98.5) (width 0.5) (layer B.Cu) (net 19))
 (segment (start 167.25 105.04) (end 167.46 105.25) (width 1) (layer B.Cu) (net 20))
 (segment (start 167.46 105.25) (end 167.46 102.96) (width 0.75) (layer B.Cu) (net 20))
 (segment (start 167.25 102.75) (end 167.25 100.5) (width 0.75) (layer B.Cu) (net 20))
 (segment (start 167.46 102.96) (end 167.25 102.75) (width 0.75) (layer B.Cu) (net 20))
 (segment (start 167.25 98.5) (end 167.25 100.5) (width 0.5) (layer B.Cu) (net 20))
 (segment (start 168 97.75) (end 167.25 98.5) (width 0.5) (layer B.Cu) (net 20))
 (segment (start 168 92.37) (end 168 97.75) (width 0.5) (layer B.Cu) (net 20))
 (segment (start 170 105.25) (end 170 103.25) (width 0.75) (layer B.Cu) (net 10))
 (segment (start 169.25 102.5) (end 169.25 100.5) (width 0.75) (layer B.Cu) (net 10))
 (segment (start 170 103.25) (end 169.25 102.5) (width 0.75) (layer B.Cu) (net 10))
 (segment (start 171.25 92.37) (end 171.25 97) (width 0.5) (layer B.Cu) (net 10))
 (segment (start 169.25 99) (end 169.25 100.5) (width 0.5) (layer B.Cu) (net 10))
 (segment (start 171.25 97) (end 169.25 99) (width 0.5) (layer B.Cu) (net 10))
 (segment (start 171.25 101.675) (end 172.25 102.675) (width 0.5) (layer B.Cu) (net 9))
 (segment (start 171.25 100.5) (end 171.25 101.675) (width 0.5) (layer B.Cu) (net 9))
 (segment (start 172.25 102.675) (end 172.25 106.5) (width 0.5) (layer B.Cu) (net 9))
 (segment (start 172.25 106.5) (end 170.75 108) (width 0.5) (layer B.Cu) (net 9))
 (segment (start 170.75 108) (end 151 108) (width 0.5) (layer B.Cu) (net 9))
 (segment (start 149.5 106.5) (end 149.5 100.5) (width 0.5) (layer B.Cu) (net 9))
 (segment (start 151 108) (end 149.5 106.5) (width 0.5) (layer B.Cu) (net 9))
 (segment (start 130.5 100.5) (end 130.5 100.75) (width 0.5) (layer B.Cu) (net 9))
 (segment (start 130.5 100.75) (end 126.25 105) (width 0.5) (layer B.Cu) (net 9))
 (segment (start 126.25 105) (end 126.25 106.5) (width 0.5) (layer B.Cu) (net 9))
 (segment (start 126.25 106.5) (end 127.75 108) (width 0.5) (layer B.Cu) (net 9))
 (segment (start 148 108) (end 149.5 106.5) (width 0.5) (layer B.Cu) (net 9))
 (segment (start 127.75 108) (end 148 108) (width 0.5) (layer B.Cu) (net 9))
 (segment (start 121.25 101.454594) (end 120.204594 102.5) (width 0.5) (layer B.Cu) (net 9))
 (segment (start 121.25 100.5) (end 121.25 101.454594) (width 0.5) (layer B.Cu) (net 9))
 (segment (start 120.204594 102.5) (end 119.5 102.5) (width 0.5) (layer B.Cu) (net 9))
 (segment (start 119.5 102.5) (end 118.75 103.25) (width 0.5) (layer B.Cu) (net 9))
 (segment (start 118.75 103.25) (end 118.75 106.5) (width 0.5) (layer B.Cu) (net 9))
 (segment (start 118.75 106.5) (end 120.25 108) (width 0.5) (layer B.Cu) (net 9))
 (segment (start 124.75 108) (end 126.25 106.5) (width 0.5) (layer B.Cu) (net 9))
 (segment (start 120.25 108) (end 124.75 108) (width 0.5) (layer B.Cu) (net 9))
 (segment (start 122.75 84.75) (end 171.25 84.75) (width 0.5) (layer B.Cu) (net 9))
 (segment (start 171.25 99.325) (end 173.25 97.325) (width 0.5) (layer B.Cu) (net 9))
 (segment (start 171.25 100.5) (end 171.25 99.325) (width 0.5) (layer B.Cu) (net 9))
 (segment (start 173.25 86.75) (end 171.25 84.75) (width 0.5) (layer B.Cu) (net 9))
 (segment (start 173.25 97.325) (end 173.25 86.75) (width 0.5) (layer B.Cu) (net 9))
 (segment (start 158.25 77.25) (end 158.5 77) (width 0.5) (layer B.Cu) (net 9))
 (segment (start 158.25 84.75) (end 158.25 77.25) (width 0.5) (layer B.Cu) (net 9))
 (segment (start 139 77) (end 145 77) (width 0.5) (layer B.Cu) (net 9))
 (segment (start 145 77) (end 147 75) (width 0.5) (layer B.Cu) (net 9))
 (segment (start 156.5 75) (end 158.5 77) (width 0.5) (layer B.Cu) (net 9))
 (segment (start 147 75) (end 156.5 75) (width 0.5) (layer B.Cu) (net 9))
 (segment (start 133.5 101.454594) (end 132.704594 102.25) (width 0.5) (layer B.Cu) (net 1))
 (segment (start 133.5 100.5) (end 133.5 101.454594) (width 0.5) (layer B.Cu) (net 1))
 (segment (start 131.72 102.25) (end 128.72 105.25) (width 0.5) (layer B.Cu) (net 1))
 (segment (start 132.704594 102.25) (end 131.72 102.25) (width 0.5) (layer B.Cu) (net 1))
 (segment (start 133.5 99.545406) (end 131.204594 97.25) (width 0.5) (layer B.Cu) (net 1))
 (segment (start 133.5 100.5) (end 133.5 99.545406) (width 0.5) (layer B.Cu) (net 1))
 (segment (start 127.63 97.25) (end 122.75 92.37) (width 0.5) (layer B.Cu) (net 1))
 (segment (start 131.204594 97.25) (end 127.63 97.25) (width 0.5) (layer B.Cu) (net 1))
 (segment (start 133.26 103.25) (end 131.26 105.25) (width 0.5) (layer B.Cu) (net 2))
 (segment (start 134 103.25) (end 133.26 103.25) (width 0.5) (layer B.Cu) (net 2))
 (segment (start 135.5 101.75) (end 134 103.25) (width 0.5) (layer B.Cu) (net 2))
 (segment (start 135.5 100.5) (end 135.5 101.75) (width 0.5) (layer B.Cu) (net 2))
 (segment (start 129.63 96) (end 126 92.37) (width 0.5) (layer B.Cu) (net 2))
 (segment (start 132 96) (end 129.63 96) (width 0.5) (layer B.Cu) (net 2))
 (segment (start 135.5 99.5) (end 132 96) (width 0.5) (layer B.Cu) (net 2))
 (segment (start 135.5 100.5) (end 135.5 99.5) (width 0.5) (layer B.Cu) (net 2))
 (segment (start 136.25 102.75) (end 137.5 101.5) (width 0.5) (layer B.Cu) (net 3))
 (segment (start 137.5 101.5) (end 137.5 100.5) (width 0.5) (layer B.Cu) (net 3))
 (segment (start 133.8 105.25) (end 136.25 102.75) (width 0.5) (layer B.Cu) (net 3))
 (segment (start 137.5 99.545406) (end 132.704594 94.75) (width 0.5) (layer B.Cu) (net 3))
 (segment (start 137.5 100.5) (end 137.5 99.545406) (width 0.5) (layer B.Cu) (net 3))
 (segment (start 131.63 94.75) (end 129.25 92.37) (width 0.5) (layer B.Cu) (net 3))
 (segment (start 132.704594 94.75) (end 131.63 94.75) (width 0.5) (layer B.Cu) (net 3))
 (segment (start 137.25 104) (end 139.5 101.75) (width 0.5) (layer B.Cu) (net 4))
 (segment (start 139.5 101.75) (end 139.5 100.5) (width 0.5) (layer B.Cu) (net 4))
 (segment (start 136.34 105.25) (end 137.25 104) (width 0.5) (layer B.Cu) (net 4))
 (segment (start 139.5 99.37) (end 132.5 92.37) (width 0.5) (layer B.Cu) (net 4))
 (segment (start 139.5 100.5) (end 139.5 99.37) (width 0.5) (layer B.Cu) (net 4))
 (segment (start 141.5 101.49863) (end 141.5 100.5) (width 0.5) (layer B.Cu) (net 5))
 (segment (start 138.88 104.11863) (end 141.5 101.49863) (width 0.5) (layer B.Cu) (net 5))
 (segment (start 138.88 105.25) (end 138.88 104.11863) (width 0.5) (layer B.Cu) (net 5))
 (segment (start 141.5 98.12) (end 135.75 92.37) (width 0.5) (layer B.Cu) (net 5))
 (segment (start 141.5 100.5) (end 141.5 98.12) (width 0.5) (layer B.Cu) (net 5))
 (segment (start 141.42 105.25) (end 141.42 104.08) (width 0.5) (layer B.Cu) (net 6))
 (segment (start 143.5 102) (end 143.5 100.5) (width 0.5) (layer B.Cu) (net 6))
 (segment (start 141.42 104.08) (end 143.5 102) (width 0.5) (layer B.Cu) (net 6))
 (segment (start 143.5 96.87) (end 139 92.37) (width 0.5) (layer B.Cu) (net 6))
 (segment (start 143.5 100.5) (end 143.5 96.87) (width 0.5) (layer B.Cu) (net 6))
 (segment (start 143.96 104.11863) (end 145.5 102.57863) (width 0.5) (layer B.Cu) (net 7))
 (segment (start 143.96 105.25) (end 143.96 104.11863) (width 0.5) (layer B.Cu) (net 7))
 (segment (start 145.5 102.57863) (end 145.5 100.5) (width 0.5) (layer B.Cu) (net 7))
 (segment (start 145.5 100.5) (end 145.5 96.75) (width 0.5) (layer B.Cu) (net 7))
 (segment (start 145.5 96.75) (end 142.25 93.5) (width 0.5) (layer B.Cu) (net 7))
 (segment (start 142.25 93.5) (end 142.25 92.37) (width 0.5) (layer B.Cu) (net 7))
 (segment (start 146.5 105.25) (end 147.5 104.25) (width 0.5) (layer B.Cu) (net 8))
 (segment (start 147.5 104.25) (end 147.5 100.5) (width 0.5) (layer B.Cu) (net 8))
 (segment (start 147.5 100.5) (end 147.5 96) (width 0.5) (layer B.Cu) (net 8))
 (segment (start 145.25 93.75) (end 145.25 92.37) (width 0.5) (layer B.Cu) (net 8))
 (segment (start 147.5 96) (end 145.25 93.75) (width 0.5) (layer B.Cu) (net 8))
 (segment (start 123.75 103.5) (end 126.5 100.5) (width 0.5) (layer B.Cu) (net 12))
 (segment (start 120.46 104.11863) (end 121.07863 103.5) (width 0.5) (layer B.Cu) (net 12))
 (segment (start 121.07863 103.5) (end 123.75 103.5) (width 0.5) (layer B.Cu) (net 12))
 (segment (start 120.46 105.25) (end 120.46 104.11863) (width 0.5) (layer B.Cu) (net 12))
 (segment (start 118.5 82) (end 123.5 77) (width 0.5) (layer B.Cu) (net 12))
 (segment (start 123.5 77) (end 131.38 77) (width 0.5) (layer B.Cu) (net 12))
 (segment (start 118.5 93.5) (end 118.5 82) (width 0.5) (layer B.Cu) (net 12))
 (segment (start 120.25 95.25) (end 118.5 93.5) (width 0.5) (layer B.Cu) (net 12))
 (segment (start 121.25 95.25) (end 120.25 95.25) (width 0.5) (layer B.Cu) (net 12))
 (segment (start 126.5 100.5) (end 121.25 95.25) (width 0.5) (layer B.Cu) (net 12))
 (segment (start 126.75 102.5) (end 128.5 100.5) (width 0.5) (layer B.Cu) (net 13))
 (segment (start 124.25 105.25) (end 126.75 102.5) (width 0.5) (layer B.Cu) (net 13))
 (segment (start 123 105.25) (end 124.25 105.25) (width 0.5) (layer B.Cu) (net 13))
 (segment (start 150.88 79.12) (end 150.88 77) (width 0.5) (layer B.Cu) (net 13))
 (segment (start 149 81) (end 150.88 79.12) (width 0.5) (layer B.Cu) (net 13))
 (segment (start 122.5 81) (end 149 81) (width 0.5) (layer B.Cu) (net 13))
 (segment (start 120 92.75) (end 120 83.5) (width 0.5) (layer B.Cu) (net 13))
 (segment (start 121.25 94) (end 120 92.75) (width 0.5) (layer B.Cu) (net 13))
 (segment (start 120 83.5) (end 122.5 81) (width 0.5) (layer B.Cu) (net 13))
 (segment (start 122.25 94) (end 121.25 94) (width 0.5) (layer B.Cu) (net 13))
 (segment (start 128 98.5) (end 126.75 98.5) (width 0.5) (layer B.Cu) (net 13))
 (segment (start 126.75 98.5) (end 122.25 94) (width 0.5) (layer B.Cu) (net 13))
 (segment (start 128.5 99) (end 128 98.5) (width 0.5) (layer B.Cu) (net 13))
 (segment (start 128.5 100.5) (end 128.5 99) (width 0.5) (layer B.Cu) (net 13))
 (segment (start 128.72 112.87) (end 170 112.87) (width 1) (layer B.Cu) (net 11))
 (segment (start 120.46 112.87) (end 128.72 112.87) (width 1) (layer B.Cu) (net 11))
 (segment (start 117.825 100.5) (end 117 101.325) (width 0.5) (layer B.Cu) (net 11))
 (segment (start 119.25 100.5) (end 118.075 100.5) (width 0.5) (layer B.Cu) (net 11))
 (segment (start 117 101.325) (end 117 112) (width 0.5) (layer B.Cu) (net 11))
 (segment (start 118.12 112.87) (end 120.46 112.87) (width 0.5) (layer B.Cu) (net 11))
 (segment (start 117 112) (end 117.87 112.87) (width 0.5) (layer B.Cu) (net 11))
 (segment (start 123.25 100.5) (end 123.25 99.25) (width 0.5) (layer B.Cu) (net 11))
 (segment (start 123.25 99.25) (end 122.5 98.5) (width 0.5) (layer B.Cu) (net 11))
 (segment (start 119.25 99.325) (end 119.25 100.5) (width 0.5) (layer B.Cu) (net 11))
 (segment (start 120.075 98.5) (end 119.25 99.325) (width 0.5) (layer B.Cu) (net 11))
 (segment (start 122.5 98.5) (end 120.075 98.5) (width 0.5) (layer B.Cu) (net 11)))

